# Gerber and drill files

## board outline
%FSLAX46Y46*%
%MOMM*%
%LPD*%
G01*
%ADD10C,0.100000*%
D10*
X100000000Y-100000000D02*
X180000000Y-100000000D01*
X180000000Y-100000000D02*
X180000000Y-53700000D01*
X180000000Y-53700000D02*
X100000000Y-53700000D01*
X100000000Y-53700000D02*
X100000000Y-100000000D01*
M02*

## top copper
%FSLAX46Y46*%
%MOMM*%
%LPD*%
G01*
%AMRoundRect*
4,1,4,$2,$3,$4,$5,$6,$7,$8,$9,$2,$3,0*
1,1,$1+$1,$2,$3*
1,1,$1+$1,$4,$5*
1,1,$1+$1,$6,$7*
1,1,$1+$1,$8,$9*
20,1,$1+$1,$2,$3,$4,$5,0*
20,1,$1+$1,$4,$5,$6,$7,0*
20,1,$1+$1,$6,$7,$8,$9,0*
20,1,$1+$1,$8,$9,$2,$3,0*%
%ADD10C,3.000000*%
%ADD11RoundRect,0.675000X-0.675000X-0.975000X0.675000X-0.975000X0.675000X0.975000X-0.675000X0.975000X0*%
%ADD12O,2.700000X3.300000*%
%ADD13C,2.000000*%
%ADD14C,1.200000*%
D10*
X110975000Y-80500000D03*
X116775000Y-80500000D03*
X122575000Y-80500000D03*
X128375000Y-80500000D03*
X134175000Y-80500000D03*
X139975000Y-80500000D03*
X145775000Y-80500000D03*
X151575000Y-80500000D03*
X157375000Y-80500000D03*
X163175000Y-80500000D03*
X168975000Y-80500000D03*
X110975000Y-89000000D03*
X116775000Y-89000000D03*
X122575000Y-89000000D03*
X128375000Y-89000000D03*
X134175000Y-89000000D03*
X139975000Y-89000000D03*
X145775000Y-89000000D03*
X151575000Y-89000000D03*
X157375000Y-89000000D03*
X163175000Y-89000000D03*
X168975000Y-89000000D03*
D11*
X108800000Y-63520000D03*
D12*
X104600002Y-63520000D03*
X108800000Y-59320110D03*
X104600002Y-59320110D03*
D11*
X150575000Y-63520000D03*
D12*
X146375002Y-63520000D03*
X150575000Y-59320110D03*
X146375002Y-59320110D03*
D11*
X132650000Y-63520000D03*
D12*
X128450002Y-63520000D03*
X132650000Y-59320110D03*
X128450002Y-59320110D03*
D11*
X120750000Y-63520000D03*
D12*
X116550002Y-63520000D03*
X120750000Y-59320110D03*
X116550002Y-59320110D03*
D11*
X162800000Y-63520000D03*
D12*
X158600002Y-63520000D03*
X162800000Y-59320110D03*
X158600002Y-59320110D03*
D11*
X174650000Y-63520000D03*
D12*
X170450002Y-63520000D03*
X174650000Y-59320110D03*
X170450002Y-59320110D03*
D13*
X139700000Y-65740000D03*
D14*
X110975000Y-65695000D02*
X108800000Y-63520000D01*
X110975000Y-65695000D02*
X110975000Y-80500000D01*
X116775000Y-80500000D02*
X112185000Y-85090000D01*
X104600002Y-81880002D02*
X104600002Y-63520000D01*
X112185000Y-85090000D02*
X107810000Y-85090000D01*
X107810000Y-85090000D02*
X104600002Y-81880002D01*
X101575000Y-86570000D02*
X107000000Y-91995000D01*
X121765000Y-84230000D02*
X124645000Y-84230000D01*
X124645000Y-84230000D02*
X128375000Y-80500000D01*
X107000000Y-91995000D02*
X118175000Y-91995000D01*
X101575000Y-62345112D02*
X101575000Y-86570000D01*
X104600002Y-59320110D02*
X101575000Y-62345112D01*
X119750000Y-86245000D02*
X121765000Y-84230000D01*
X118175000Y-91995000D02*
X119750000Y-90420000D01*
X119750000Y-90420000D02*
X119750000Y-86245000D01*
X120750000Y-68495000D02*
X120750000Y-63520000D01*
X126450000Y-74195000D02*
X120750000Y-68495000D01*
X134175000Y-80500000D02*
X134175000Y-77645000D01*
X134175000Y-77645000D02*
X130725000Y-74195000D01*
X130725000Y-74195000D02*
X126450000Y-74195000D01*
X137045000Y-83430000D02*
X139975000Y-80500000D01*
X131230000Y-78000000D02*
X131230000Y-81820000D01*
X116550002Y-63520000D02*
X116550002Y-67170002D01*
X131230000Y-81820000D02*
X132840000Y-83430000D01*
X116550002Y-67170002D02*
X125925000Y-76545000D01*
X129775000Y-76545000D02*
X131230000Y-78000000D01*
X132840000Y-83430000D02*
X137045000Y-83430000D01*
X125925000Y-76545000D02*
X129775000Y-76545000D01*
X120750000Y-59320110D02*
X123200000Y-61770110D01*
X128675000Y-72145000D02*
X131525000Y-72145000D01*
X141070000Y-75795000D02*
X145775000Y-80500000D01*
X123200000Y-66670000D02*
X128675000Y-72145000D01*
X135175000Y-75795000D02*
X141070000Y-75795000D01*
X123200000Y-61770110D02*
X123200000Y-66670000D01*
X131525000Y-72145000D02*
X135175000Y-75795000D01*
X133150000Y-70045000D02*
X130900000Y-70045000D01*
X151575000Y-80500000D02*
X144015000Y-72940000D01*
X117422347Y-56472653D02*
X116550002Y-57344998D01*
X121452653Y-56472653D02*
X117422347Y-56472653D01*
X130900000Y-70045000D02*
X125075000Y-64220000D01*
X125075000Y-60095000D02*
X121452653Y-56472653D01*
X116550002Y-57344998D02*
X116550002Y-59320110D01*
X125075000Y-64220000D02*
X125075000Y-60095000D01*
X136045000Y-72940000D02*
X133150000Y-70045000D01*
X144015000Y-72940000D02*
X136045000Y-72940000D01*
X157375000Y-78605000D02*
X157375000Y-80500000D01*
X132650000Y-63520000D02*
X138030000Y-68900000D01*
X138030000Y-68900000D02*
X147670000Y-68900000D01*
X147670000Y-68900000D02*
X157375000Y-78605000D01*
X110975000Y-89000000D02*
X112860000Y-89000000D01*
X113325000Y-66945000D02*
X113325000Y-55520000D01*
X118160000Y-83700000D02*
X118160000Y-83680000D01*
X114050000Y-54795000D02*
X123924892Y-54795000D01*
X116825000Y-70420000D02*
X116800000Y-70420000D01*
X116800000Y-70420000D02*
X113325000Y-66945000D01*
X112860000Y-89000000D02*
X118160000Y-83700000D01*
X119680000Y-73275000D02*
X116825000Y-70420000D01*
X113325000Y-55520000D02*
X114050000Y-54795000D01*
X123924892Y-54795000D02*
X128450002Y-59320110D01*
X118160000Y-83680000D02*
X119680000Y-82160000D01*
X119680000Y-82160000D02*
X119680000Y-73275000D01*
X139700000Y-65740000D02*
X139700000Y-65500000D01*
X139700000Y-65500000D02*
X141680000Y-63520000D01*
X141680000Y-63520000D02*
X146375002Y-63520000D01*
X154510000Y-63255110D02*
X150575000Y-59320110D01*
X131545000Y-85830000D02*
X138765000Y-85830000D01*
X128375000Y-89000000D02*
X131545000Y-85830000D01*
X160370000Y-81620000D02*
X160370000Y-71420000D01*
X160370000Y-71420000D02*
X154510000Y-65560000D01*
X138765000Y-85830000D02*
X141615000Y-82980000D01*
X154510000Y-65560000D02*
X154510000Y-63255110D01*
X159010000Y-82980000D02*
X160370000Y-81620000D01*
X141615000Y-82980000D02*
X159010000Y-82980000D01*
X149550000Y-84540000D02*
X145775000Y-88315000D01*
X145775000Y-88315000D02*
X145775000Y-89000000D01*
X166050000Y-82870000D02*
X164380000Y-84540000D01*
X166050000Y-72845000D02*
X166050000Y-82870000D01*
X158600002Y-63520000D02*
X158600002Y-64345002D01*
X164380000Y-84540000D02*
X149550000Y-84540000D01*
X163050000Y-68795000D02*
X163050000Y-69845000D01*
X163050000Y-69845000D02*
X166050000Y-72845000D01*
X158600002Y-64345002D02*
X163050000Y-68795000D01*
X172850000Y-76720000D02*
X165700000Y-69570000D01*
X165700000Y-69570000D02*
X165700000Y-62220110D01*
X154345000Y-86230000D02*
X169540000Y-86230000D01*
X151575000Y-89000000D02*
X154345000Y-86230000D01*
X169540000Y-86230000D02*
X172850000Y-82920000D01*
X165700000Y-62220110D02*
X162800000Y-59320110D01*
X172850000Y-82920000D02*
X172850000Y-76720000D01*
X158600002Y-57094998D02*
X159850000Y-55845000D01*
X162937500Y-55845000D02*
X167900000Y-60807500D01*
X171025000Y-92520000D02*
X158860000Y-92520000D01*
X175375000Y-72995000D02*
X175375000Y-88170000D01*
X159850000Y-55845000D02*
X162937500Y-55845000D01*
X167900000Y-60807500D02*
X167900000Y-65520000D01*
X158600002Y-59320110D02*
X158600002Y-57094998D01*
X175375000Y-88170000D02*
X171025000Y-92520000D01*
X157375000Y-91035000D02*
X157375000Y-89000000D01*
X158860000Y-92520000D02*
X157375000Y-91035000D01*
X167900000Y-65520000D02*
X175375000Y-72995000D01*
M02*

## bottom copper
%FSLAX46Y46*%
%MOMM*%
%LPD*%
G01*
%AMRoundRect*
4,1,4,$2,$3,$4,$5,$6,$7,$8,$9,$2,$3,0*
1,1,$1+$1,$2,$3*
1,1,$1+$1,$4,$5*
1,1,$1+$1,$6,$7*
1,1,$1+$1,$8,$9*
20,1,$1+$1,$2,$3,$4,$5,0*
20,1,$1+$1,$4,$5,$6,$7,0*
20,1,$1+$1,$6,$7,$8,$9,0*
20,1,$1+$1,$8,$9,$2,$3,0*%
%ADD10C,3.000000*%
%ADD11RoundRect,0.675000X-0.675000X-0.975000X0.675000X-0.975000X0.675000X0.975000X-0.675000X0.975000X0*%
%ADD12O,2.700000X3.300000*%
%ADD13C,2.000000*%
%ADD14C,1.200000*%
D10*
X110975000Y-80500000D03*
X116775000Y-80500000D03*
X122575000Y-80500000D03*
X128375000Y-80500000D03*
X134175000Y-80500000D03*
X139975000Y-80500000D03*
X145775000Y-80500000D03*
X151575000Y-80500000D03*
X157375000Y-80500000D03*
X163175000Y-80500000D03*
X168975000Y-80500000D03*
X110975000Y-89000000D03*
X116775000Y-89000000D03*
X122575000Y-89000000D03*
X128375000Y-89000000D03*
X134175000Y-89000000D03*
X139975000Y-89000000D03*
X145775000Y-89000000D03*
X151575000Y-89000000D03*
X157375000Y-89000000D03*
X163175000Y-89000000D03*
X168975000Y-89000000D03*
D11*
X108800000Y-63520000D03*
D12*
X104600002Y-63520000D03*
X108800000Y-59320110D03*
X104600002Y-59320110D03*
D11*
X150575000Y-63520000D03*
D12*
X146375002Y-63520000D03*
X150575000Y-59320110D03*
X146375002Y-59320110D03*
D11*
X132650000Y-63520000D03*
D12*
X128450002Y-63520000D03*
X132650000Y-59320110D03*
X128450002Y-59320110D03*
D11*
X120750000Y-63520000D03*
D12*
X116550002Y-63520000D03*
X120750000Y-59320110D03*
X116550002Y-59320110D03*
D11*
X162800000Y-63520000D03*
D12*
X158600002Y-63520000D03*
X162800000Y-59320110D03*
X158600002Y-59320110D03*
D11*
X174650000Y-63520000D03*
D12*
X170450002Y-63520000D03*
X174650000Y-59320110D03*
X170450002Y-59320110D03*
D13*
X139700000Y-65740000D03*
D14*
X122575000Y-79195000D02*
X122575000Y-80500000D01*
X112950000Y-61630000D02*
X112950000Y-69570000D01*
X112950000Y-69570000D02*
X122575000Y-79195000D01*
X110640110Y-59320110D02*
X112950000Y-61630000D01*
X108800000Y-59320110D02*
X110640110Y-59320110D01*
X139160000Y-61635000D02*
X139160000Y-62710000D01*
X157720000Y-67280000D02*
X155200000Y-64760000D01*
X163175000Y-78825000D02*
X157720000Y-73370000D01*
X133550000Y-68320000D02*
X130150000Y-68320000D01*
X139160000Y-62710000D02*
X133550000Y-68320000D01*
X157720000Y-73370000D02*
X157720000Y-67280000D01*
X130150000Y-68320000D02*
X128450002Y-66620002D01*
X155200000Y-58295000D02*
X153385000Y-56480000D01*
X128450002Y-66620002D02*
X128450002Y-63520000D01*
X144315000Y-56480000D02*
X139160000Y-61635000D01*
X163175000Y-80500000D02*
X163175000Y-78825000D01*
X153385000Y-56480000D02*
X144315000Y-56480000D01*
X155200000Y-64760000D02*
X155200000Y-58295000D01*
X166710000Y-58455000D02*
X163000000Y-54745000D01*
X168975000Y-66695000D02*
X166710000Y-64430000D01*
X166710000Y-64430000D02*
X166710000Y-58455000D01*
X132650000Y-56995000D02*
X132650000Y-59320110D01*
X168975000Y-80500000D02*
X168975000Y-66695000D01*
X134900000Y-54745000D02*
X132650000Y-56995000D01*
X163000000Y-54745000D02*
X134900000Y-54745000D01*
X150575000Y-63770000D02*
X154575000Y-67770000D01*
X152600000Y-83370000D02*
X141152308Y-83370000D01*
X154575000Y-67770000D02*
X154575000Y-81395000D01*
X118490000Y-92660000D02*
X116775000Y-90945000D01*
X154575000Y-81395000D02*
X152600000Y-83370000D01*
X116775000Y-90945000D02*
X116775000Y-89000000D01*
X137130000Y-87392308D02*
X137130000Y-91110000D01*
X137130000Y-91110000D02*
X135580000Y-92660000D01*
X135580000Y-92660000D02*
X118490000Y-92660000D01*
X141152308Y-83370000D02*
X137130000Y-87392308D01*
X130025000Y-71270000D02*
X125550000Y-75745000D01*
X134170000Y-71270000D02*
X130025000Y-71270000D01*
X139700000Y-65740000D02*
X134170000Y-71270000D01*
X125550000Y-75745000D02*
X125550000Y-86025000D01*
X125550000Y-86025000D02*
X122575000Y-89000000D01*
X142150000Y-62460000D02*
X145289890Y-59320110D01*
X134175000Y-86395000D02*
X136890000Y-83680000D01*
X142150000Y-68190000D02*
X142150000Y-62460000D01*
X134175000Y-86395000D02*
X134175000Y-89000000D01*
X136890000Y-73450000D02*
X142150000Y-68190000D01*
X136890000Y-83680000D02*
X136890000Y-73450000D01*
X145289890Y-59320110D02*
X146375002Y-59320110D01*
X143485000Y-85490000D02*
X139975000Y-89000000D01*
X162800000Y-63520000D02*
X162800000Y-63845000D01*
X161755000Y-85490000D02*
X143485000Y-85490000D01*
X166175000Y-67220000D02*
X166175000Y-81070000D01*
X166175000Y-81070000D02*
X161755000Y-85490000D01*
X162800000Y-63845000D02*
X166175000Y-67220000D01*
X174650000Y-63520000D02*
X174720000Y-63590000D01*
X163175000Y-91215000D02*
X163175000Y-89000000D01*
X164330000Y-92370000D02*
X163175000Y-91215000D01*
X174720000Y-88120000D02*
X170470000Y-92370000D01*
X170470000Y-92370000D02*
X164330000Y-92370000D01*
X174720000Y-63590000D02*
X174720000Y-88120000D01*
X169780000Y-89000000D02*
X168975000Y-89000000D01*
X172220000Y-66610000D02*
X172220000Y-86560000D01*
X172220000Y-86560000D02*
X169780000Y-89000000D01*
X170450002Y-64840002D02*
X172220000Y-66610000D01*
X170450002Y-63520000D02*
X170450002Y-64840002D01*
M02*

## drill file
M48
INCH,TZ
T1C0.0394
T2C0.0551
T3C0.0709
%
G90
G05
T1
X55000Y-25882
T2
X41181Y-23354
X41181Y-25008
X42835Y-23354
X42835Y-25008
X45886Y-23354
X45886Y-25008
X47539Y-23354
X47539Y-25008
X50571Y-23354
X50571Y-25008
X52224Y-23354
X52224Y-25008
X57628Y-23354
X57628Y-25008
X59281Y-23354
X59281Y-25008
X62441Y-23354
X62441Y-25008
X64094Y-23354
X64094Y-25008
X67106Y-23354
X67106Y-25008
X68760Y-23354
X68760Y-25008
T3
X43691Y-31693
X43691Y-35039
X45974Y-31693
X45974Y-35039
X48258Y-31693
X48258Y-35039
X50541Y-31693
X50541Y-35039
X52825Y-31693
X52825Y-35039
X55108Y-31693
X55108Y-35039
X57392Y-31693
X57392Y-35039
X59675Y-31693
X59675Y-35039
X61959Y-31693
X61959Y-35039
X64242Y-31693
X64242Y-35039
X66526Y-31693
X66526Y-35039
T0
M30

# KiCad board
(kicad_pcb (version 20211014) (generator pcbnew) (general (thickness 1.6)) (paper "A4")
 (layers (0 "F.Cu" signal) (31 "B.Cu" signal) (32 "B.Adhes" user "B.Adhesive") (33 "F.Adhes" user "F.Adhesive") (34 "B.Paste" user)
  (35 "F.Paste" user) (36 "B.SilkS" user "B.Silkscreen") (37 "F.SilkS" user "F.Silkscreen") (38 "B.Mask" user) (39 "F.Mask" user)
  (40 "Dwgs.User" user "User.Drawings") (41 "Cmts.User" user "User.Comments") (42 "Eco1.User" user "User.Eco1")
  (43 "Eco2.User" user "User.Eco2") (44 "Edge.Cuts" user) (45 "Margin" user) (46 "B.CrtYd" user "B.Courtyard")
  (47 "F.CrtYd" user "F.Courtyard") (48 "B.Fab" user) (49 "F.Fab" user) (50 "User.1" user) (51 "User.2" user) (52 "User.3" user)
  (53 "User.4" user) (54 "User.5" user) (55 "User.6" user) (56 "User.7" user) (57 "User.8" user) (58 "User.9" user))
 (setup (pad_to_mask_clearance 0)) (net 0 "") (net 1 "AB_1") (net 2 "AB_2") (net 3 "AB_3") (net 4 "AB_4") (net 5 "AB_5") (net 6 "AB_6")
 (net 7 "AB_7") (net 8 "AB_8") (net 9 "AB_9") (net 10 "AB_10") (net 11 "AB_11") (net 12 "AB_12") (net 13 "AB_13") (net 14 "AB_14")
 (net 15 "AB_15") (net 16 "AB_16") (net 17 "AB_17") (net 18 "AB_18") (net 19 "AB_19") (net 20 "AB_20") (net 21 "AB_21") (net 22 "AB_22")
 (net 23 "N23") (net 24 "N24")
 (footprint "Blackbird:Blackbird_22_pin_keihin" (layer "F.Cu") (at 110.975 80.5)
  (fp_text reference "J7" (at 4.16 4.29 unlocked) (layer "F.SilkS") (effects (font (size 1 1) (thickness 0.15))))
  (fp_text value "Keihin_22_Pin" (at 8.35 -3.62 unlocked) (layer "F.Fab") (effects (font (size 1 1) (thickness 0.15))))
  (pad "1" thru_hole circle (at 0 0) (size 3 3) (drill 1.8) (layers *.Cu *.Mask) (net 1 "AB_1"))
  (pad "2" thru_hole circle (at 5.8 0) (size 3 3) (drill 1.8) (layers *.Cu *.Mask) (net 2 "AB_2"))
  (pad "3" thru_hole circle (at 11.6 0) (size 3 3) (drill 1.8) (layers *.Cu *.Mask) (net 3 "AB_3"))
  (pad "4" thru_hole circle (at 17.4 0) (size 3 3) (drill 1.8) (layers *.Cu *.Mask) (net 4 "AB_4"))
  (pad "5" thru_hole circle (at 23.2 0) (size 3 3) (drill 1.8) (layers *.Cu *.Mask) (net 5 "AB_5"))
  (pad "6" thru_hole circle (at 29 0) (size 3 3) (drill 1.8) (layers *.Cu *.Mask) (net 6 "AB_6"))
  (pad "7" thru_hole circle (at 34.8 0) (size 3 3) (drill 1.8) (layers *.Cu *.Mask) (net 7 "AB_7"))
  (pad "8" thru_hole circle (at 40.6 0) (size 3 3) (drill 1.8) (layers *.Cu *.Mask) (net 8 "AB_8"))
  (pad "9" thru_hole circle (at 46.4 0) (size 3 3) (drill 1.8) (layers *.Cu *.Mask) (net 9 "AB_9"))
  (pad "10" thru_hole circle (at 52.2 0) (size 3 3) (drill 1.8) (layers *.Cu *.Mask) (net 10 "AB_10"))
  (pad "11" thru_hole circle (at 58 0) (size 3 3) (drill 1.8) (layers *.Cu *.Mask) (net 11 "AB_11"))
  (pad "12" thru_hole circle (at 0 8.5) (size 3 3) (drill 1.8) (layers *.Cu *.Mask) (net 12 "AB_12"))
  (pad "13" thru_hole circle (at 5.8 8.5) (size 3 3) (drill 1.8) (layers *.Cu *.Mask) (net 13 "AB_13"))
  (pad "14" thru_hole circle (at 11.6 8.5) (size 3 3) (drill 1.8) (layers *.Cu *.Mask) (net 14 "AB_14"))
  (pad "15" thru_hole circle (at 17.4 8.5) (size 3 3) (drill 1.8) (layers *.Cu *.Mask) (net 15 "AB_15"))
  (pad "16" thru_hole circle (at 23.2 8.5) (size 3 3) (drill 1.8) (layers *.Cu *.Mask) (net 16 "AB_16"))
  (pad "17" thru_hole circle (at 29 8.5) (size 3 3) (drill 1.8) (layers *.Cu *.Mask) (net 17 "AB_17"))
  (pad "18" thru_hole circle (at 34.8 8.5) (size 3 3) (drill 1.8) (layers *.Cu *.Mask) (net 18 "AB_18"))
  (pad "19" thru_hole circle (at 40.6 8.5) (size 3 3) (drill 1.8) (layers *.Cu *.Mask) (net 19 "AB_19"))
  (pad "20" thru_hole circle (at 46.4 8.5) (size 3 3) (drill 1.8) (layers *.Cu *.Mask) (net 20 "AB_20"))
  (pad "21" thru_hole circle (at 52.2 8.5) (size 3 3) (drill 1.8) (layers *.Cu *.Mask) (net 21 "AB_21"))
  (pad "22" thru_hole circle (at 58 8.5) (size 3 3) (drill 1.8) (layers *.Cu *.Mask) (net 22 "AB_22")))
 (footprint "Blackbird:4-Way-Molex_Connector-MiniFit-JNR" (layer "F.Cu") (at 108.8 63.52)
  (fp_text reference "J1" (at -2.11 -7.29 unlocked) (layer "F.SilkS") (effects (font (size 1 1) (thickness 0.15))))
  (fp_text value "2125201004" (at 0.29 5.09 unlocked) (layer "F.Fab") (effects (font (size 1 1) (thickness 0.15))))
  (pad "1" thru_hole roundrect (at 0 0) (size 2.7 3.3) (drill 1.4) (layers *.Cu *.Mask) (roundrect_rratio 0.25) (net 1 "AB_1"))
  (pad "2" thru_hole oval (at -4.199998 0) (size 2.7 3.3) (drill 1.4) (layers *.Cu *.Mask) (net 2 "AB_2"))
  (pad "3" thru_hole oval (at 0 -4.19989) (size 2.7 3.3) (drill 1.4) (layers *.Cu *.Mask) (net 3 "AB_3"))
  (pad "4" thru_hole oval (at -4.199998 -4.19989) (size 2.7 3.3) (drill 1.4) (layers *.Cu *.Mask) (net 4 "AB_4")))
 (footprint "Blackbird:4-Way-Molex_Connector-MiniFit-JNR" (layer "F.Cu") (at 150.575 63.52)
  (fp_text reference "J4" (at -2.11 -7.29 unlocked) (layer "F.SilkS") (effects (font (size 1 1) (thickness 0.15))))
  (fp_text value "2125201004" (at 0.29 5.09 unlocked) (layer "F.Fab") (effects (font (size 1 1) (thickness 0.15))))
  (pad "1" thru_hole roundrect (at 0 0) (size 2.7 3.3) (drill 1.4) (layers *.Cu *.Mask) (roundrect_rratio 0.25) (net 13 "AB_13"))
  (pad "2" thru_hole oval (at -4.199998 0) (size 2.7 3.3) (drill 1.4) (layers *.Cu *.Mask) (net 14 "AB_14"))
  (pad "3" thru_hole oval (at 0 -4.19989) (size 2.7 3.3) (drill 1.4) (layers *.Cu *.Mask) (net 15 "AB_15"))
  (pad "4" thru_hole oval (at -4.199998 -4.19989) (size 2.7 3.3) (drill 1.4) (layers *.Cu *.Mask) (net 16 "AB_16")))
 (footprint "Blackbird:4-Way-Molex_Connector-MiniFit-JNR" (layer "F.Cu") (at 132.65 63.52)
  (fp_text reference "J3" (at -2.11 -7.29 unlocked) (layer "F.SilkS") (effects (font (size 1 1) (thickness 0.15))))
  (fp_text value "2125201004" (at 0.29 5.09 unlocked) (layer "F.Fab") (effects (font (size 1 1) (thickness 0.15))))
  (pad "1" thru_hole roundrect (at 0 0) (size 2.7 3.3) (drill 1.4) (layers *.Cu *.Mask) (roundrect_rratio 0.25) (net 9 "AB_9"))
  (pad "2" thru_hole oval (at -4.199998 0) (size 2.7 3.3) (drill 1.4) (layers *.Cu *.Mask) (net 10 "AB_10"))
  (pad "3" thru_hole oval (at 0 -4.19989) (size 2.7 3.3) (drill 1.4) (layers *.Cu *.Mask) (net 11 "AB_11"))
  (pad "4" thru_hole oval (at -4.199998 -4.19989) (size 2.7 3.3) (drill 1.4) (layers *.Cu *.Mask) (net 12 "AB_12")))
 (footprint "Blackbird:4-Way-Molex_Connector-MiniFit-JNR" (layer "F.Cu") (at 120.75 63.52)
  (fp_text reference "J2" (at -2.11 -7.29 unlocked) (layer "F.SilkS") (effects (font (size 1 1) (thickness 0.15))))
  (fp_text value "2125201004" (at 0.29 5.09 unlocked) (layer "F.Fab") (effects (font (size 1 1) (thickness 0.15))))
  (pad "1" thru_hole roundrect (at 0 0) (size 2.7 3.3) (drill 1.4) (layers *.Cu *.Mask) (roundrect_rratio 0.25) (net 5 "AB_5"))
  (pad "2" thru_hole oval (at -4.199998 0) (size 2.7 3.3) (drill 1.4) (layers *.Cu *.Mask) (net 6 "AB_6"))
  (pad "3" thru_hole oval (at 0 -4.19989) (size 2.7 3.3) (drill 1.4) (layers *.Cu *.Mask) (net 7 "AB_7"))
  (pad "4" thru_hole oval (at -4.199998 -4.19989) (size 2.7 3.3) (drill 1.4) (layers *.Cu *.Mask) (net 8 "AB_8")))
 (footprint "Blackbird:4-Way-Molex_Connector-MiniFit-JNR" (layer "F.Cu") (at 162.8 63.52)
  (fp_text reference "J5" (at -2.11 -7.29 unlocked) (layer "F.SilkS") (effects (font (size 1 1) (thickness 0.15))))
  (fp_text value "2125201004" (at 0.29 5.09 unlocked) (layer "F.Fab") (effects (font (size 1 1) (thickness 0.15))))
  (pad "1" thru_hole roundrect (at 0 0) (size 2.7 3.3) (drill 1.4) (layers *.Cu *.Mask) (roundrect_rratio 0.25) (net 17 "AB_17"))
  (pad "2" thru_hole oval (at -4.199998 0) (size 2.7 3.3) (drill 1.4) (layers *.Cu *.Mask) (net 18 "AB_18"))
  (pad "3" thru_hole oval (at 0 -4.19989) (size 2.7 3.3) (drill 1.4) (layers *.Cu *.Mask) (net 19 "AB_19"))
  (pad "4" thru_hole oval (at -4.199998 -4.19989) (size 2.7 3.3) (drill 1.4) (layers *.Cu *.Mask) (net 20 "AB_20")))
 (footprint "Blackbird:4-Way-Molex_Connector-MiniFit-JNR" (layer "F.Cu") (at 174.65 63.52)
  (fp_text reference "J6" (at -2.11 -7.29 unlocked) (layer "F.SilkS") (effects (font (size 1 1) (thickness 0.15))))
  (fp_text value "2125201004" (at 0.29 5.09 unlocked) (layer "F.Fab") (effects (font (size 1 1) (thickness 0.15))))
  (pad "1" thru_hole roundrect (at 0 0) (size 2.7 3.3) (drill 1.4) (layers *.Cu *.Mask) (roundrect_rratio 0.25) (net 21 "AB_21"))
  (pad "2" thru_hole oval (at -4.199998 0) (size 2.7 3.3) (drill 1.4) (layers *.Cu *.Mask) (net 22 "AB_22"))
  (pad "3" thru_hole oval (at 0 -4.19989) (size 2.7 3.3) (drill 1.4) (layers *.Cu *.Mask) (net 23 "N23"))
  (pad "4" thru_hole oval (at -4.199998 -4.19989) (size 2.7 3.3) (drill 1.4) (layers *.Cu *.Mask) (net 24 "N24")))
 (gr_rect (start 100 100) (end 180 53.7) (layer "Edge.Cuts") (width 0.1) (fill none))
 (segment (start 110.975 65.695) (end 108.8 63.52) (width 1.2) (layer "F.Cu") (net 1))
 (segment (start 110.975 65.695) (end 110.975 80.5) (width 1.2) (layer "F.Cu") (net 1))
 (segment (start 116.775 80.5) (end 112.185 85.09) (width 1.2) (layer "F.Cu") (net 2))
 (segment (start 104.600002 81.880002) (end 104.600002 63.52) (width 1.2) (layer "F.Cu") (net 2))
 (segment (start 112.185 85.09) (end 107.81 85.09) (width 1.2) (layer "F.Cu") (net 2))
 (segment (start 107.81 85.09) (end 104.600002 81.880002) (width 1.2) (layer "F.Cu") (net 2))
 (segment (start 122.575 79.195) (end 122.575 80.5) (width 1.2) (layer "B.Cu") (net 3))
 (segment (start 112.95 61.63) (end 112.95 69.57) (width 1.2) (layer "B.Cu") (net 3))
 (segment (start 112.95 69.57) (end 122.575 79.195) (width 1.2) (layer "B.Cu") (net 3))
 (segment (start 110.64011 59.32011) (end 112.95 61.63) (width 1.2) (layer "B.Cu") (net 3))
 (segment (start 108.8 59.32011) (end 110.64011 59.32011) (width 1.2) (layer "B.Cu") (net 3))
 (segment (start 101.575 86.57) (end 107 91.995) (width 1.2) (layer "F.Cu") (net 4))
 (segment (start 121.765 84.23) (end 124.645 84.23) (width 1.2) (layer "F.Cu") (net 4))
 (segment (start 124.645 84.23) (end 128.375 80.5) (width 1.2) (layer "F.Cu") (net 4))
 (segment (start 107 91.995) (end 118.175 91.995) (width 1.2) (layer "F.Cu") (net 4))
 (segment (start 101.575 62.345112) (end 101.575 86.57) (width 1.2) (layer "F.Cu") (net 4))
 (segment (start 104.600002 59.32011) (end 101.575 62.345112) (width 1.2) (layer "F.Cu") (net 4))
 (segment (start 119.75 86.245) (end 121.765 84.23) (width 1.2) (layer "F.Cu") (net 4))
 (segment (start 118.175 91.995) (end 119.75 90.42) (width 1.2) (layer "F.Cu") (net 4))
 (segment (start 119.75 90.42) (end 119.75 86.245) (width 1.2) (layer "F.Cu") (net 4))
 (segment (start 120.75 68.495) (end 120.75 63.52) (width 1.2) (layer "F.Cu") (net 5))
 (segment (start 126.45 74.195) (end 120.75 68.495) (width 1.2) (layer "F.Cu") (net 5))
 (segment (start 134.175 80.5) (end 134.175 77.645) (width 1.2) (layer "F.Cu") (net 5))
 (segment (start 134.175 77.645) (end 130.725 74.195) (width 1.2) (layer "F.Cu") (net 5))
 (segment (start 130.725 74.195) (end 126.45 74.195) (width 1.2) (layer "F.Cu") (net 5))
 (segment (start 137.045 83.43) (end 139.975 80.5) (width 1.2) (layer "F.Cu") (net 6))
 (segment (start 131.23 78) (end 131.23 81.82) (width 1.2) (layer "F.Cu") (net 6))
 (segment (start 116.550002 63.52) (end 116.550002 67.170002) (width 1.2) (layer "F.Cu") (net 6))
 (segment (start 131.23 81.82) (end 132.84 83.43) (width 1.2) (layer "F.Cu") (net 6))
 (segment (start 116.550002 67.170002) (end 125.925 76.545) (width 1.2) (layer "F.Cu") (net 6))
 (segment (start 129.775 76.545) (end 131.23 78) (width 1.2) (layer "F.Cu") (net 6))
 (segment (start 132.84 83.43) (end 137.045 83.43) (width 1.2) (layer "F.Cu") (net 6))
 (segment (start 125.925 76.545) (end 129.775 76.545) (width 1.2) (layer "F.Cu") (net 6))
 (segment (start 120.75 59.32011) (end 123.2 61.77011) (width 1.2) (layer "F.Cu") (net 7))
 (segment (start 128.675 72.145) (end 131.525 72.145) (width 1.2) (layer "F.Cu") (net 7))
 (segment (start 141.07 75.795) (end 145.775 80.5) (width 1.2) (layer "F.Cu") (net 7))
 (segment (start 123.2 66.67) (end 128.675 72.145) (width 1.2) (layer "F.Cu") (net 7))
 (segment (start 135.175 75.795) (end 141.07 75.795) (width 1.2) (layer "F.Cu") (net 7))
 (segment (start 123.2 61.77011) (end 123.2 66.67) (width 1.2) (layer "F.Cu") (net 7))
 (segment (start 131.525 72.145) (end 135.175 75.795) (width 1.2) (layer "F.Cu") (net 7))
 (segment (start 133.15 70.045) (end 130.9 70.045) (width 1.2) (layer "F.Cu") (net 8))
 (segment (start 151.575 80.5) (end 144.015 72.94) (width 1.2) (layer "F.Cu") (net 8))
 (segment (start 117.422347 56.472653) (end 116.550002 57.344998) (width 1.2) (layer "F.Cu") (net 8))
 (segment (start 121.452653 56.472653) (end 117.422347 56.472653) (width 1.2) (layer "F.Cu") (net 8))
 (segment (start 130.9 70.045) (end 125.075 64.22) (width 1.2) (layer "F.Cu") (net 8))
 (segment (start 125.075 60.095) (end 121.452653 56.472653) (width 1.2) (layer "F.Cu") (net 8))
 (segment (start 116.550002 57.344998) (end 116.550002 59.32011) (width 1.2) (layer "F.Cu") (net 8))
 (segment (start 125.075 64.22) (end 125.075 60.095) (width 1.2) (layer "F.Cu") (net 8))
 (segment (start 136.045 72.94) (end 133.15 70.045) (width 1.2) (layer "F.Cu") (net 8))
 (segment (start 144.015 72.94) (end 136.045 72.94) (width 1.2) (layer "F.Cu") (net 8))
 (segment (start 157.375 78.605) (end 157.375 80.5) (width 1.2) (layer "F.Cu") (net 9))
 (segment (start 132.65 63.52) (end 138.03 68.9) (width 1.2) (layer "F.Cu") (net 9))
 (segment (start 138.03 68.9) (end 147.67 68.9) (width 1.2) (layer "F.Cu") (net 9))
 (segment (start 147.67 68.9) (end 157.375 78.605) (width 1.2) (layer "F.Cu") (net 9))
 (segment (start 139.16 61.635) (end 139.16 62.71) (width 1.2) (layer "B.Cu") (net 10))
 (segment (start 157.72 67.28) (end 155.2 64.76) (width 1.2) (layer "B.Cu") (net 10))
 (segment (start 163.175 78.825) (end 157.72 73.37) (width 1.2) (layer "B.Cu") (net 10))
 (segment (start 133.55 68.32) (end 130.15 68.32) (width 1.2) (layer "B.Cu") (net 10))
 (segment (start 139.16 62.71) (end 133.55 68.32) (width 1.2) (layer "B.Cu") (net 10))
 (segment (start 157.72 73.37) (end 157.72 67.28) (width 1.2) (layer "B.Cu") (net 10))
 (segment (start 130.15 68.32) (end 128.450002 66.620002) (width 1.2) (layer "B.Cu") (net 10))
 (segment (start 155.2 58.295) (end 153.385 56.48) (width 1.2) (layer "B.Cu") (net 10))
 (segment (start 128.450002 66.620002) (end 128.450002 63.52) (width 1.2) (layer "B.Cu") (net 10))
 (segment (start 144.315 56.48) (end 139.16 61.635) (width 1.2) (layer "B.Cu") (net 10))
 (segment (start 163.175 80.5) (end 163.175 78.825) (width 1.2) (layer "B.Cu") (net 10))
 (segment (start 153.385 56.48) (end 144.315 56.48) (width 1.2) (layer "B.Cu") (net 10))
 (segment (start 155.2 64.76) (end 155.2 58.295) (width 1.2) (layer "B.Cu") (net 10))
 (segment (start 166.71 58.455) (end 163 54.745) (width 1.2) (layer "B.Cu") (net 11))
 (segment (start 168.975 66.695) (end 166.71 64.43) (width 1.2) (layer "B.Cu") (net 11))
 (segment (start 166.71 64.43) (end 166.71 58.455) (width 1.2) (layer "B.Cu") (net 11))
 (segment (start 132.65 56.995) (end 132.65 59.32011) (width 1.2) (layer "B.Cu") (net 11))
 (segment (start 168.975 80.5) (end 168.975 66.695) (width 1.2) (layer "B.Cu") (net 11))
 (segment (start 134.9 54.745) (end 132.65 56.995) (width 1.2) (layer "B.Cu") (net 11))
 (segment (start 163 54.745) (end 134.9 54.745) (width 1.2) (layer "B.Cu") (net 11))
 (segment (start 110.975 89) (end 112.86 89) (width 1.2) (layer "F.Cu") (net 12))
 (segment (start 113.325 66.945) (end 113.325 55.52) (width 1.2) (layer "F.Cu") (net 12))
 (segment (start 118.16 83.7) (end 118.16 83.68) (width 1.2) (layer "F.Cu") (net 12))
 (segment (start 114.05 54.795) (end 123.924892 54.795) (width 1.2) (layer "F.Cu") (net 12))
 (segment (start 116.825 70.42) (end 116.8 70.42) (width 1.2) (layer "F.Cu") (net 12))
 (segment (start 116.8 70.42) (end 113.325 66.945) (width 1.2) (layer "F.Cu") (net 12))
 (segment (start 112.86 89) (end 118.16 83.7) (width 1.2) (layer "F.Cu") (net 12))
 (segment (start 119.68 73.275) (end 116.825 70.42) (width 1.2) (layer "F.Cu") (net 12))
 (segment (start 113.325 55.52) (end 114.05 54.795) (width 1.2) (layer "F.Cu") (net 12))
 (segment (start 123.924892 54.795) (end 128.450002 59.32011) (width 1.2) (layer "F.Cu") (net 12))
 (segment (start 118.16 83.68) (end 119.68 82.16) (width 1.2) (layer "F.Cu") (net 12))
 (segment (start 119.68 82.16) (end 119.68 73.275) (width 1.2) (layer "F.Cu") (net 12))
 (segment (start 150.575 63.77) (end 154.575 67.77) (width 1.2) (layer "B.Cu") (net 13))
 (segment (start 152.6 83.37) (end 141.152308 83.37) (width 1.2) (layer "B.Cu") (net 13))
 (segment (start 154.575 67.77) (end 154.575 81.395) (width 1.2) (layer "B.Cu") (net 13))
 (segment (start 118.49 92.66) (end 116.775 90.945) (width 1.2) (layer "B.Cu") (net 13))
 (segment (start 154.575 81.395) (end 152.6 83.37) (width 1.2) (layer "B.Cu") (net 13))
 (segment (start 116.775 90.945) (end 116.775 89) (width 1.2) (layer "B.Cu") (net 13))
 (segment (start 137.13 87.392308) (end 137.13 91.11) (width 1.2) (layer "B.Cu") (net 13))
 (segment (start 137.13 91.11) (end 135.58 92.66) (width 1.2) (layer "B.Cu") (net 13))
 (segment (start 135.58 92.66) (end 118.49 92.66) (width 1.2) (layer "B.Cu") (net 13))
 (segment (start 141.152308 83.37) (end 137.13 87.392308) (width 1.2) (layer "B.Cu") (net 13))
 (segment (start 139.7 65.74) (end 139.7 65.5) (width 1.2) (layer "F.Cu") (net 14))
 (segment (start 139.7 65.5) (end 141.68 63.52) (width 1.2) (layer "F.Cu") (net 14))
 (segment (start 141.68 63.52) (end 146.375002 63.52) (width 1.2) (layer "F.Cu") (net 14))
 (via (at 139.7 65.74) (size 2) (drill 1) (layers "F.Cu" "B.Cu") (free) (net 14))
 (segment (start 130.025 71.27) (end 125.55 75.745) (width 1.2) (layer "B.Cu") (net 14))
 (segment (start 134.17 71.27) (end 130.025 71.27) (width 1.2) (layer "B.Cu") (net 14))
 (segment (start 139.7 65.74) (end 134.17 71.27) (width 1.2) (layer "B.Cu") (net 14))
 (segment (start 125.55 75.745) (end 125.55 86.025) (width 1.2) (layer "B.Cu") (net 14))
 (segment (start 125.55 86.025) (end 122.575 89) (width 1.2) (layer "B.Cu") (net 14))
 (segment (start 154.51 63.25511) (end 150.575 59.32011) (width 1.2) (layer "F.Cu") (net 15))
 (segment (start 131.545 85.83) (end 138.765 85.83) (width 1.2) (layer "F.Cu") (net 15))
 (segment (start 128.375 89) (end 131.545 85.83) (width 1.2) (layer "F.Cu") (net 15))
 (segment (start 160.37 81.62) (end 160.37 71.42) (width 1.2) (layer "F.Cu") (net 15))
 (segment (start 160.37 71.42) (end 154.51 65.56) (width 1.2) (layer "F.Cu") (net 15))
 (segment (start 138.765 85.83) (end 141.615 82.98) (width 1.2) (layer "F.Cu") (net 15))
 (segment (start 154.51 65.56) (end 154.51 63.25511) (width 1.2) (layer "F.Cu") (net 15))
 (segment (start 159.01 82.98) (end 160.37 81.62) (width 1.2) (layer "F.Cu") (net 15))
 (segment (start 141.615 82.98) (end 159.01 82.98) (width 1.2) (layer "F.Cu") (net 15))
 (segment (start 142.15 62.46) (end 145.28989 59.32011) (width 1.2) (layer "B.Cu") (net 16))
 (segment (start 134.175 86.395) (end 136.89 83.68) (width 1.2) (layer "B.Cu") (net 16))
 (segment (start 142.15 68.19) (end 142.15 62.46) (width 1.2) (layer "B.Cu") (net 16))
 (segment (start 134.175 86.395) (end 134.175 89) (width 1.2) (layer "B.Cu") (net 16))
 (segment (start 136.89 73.45) (end 142.15 68.19) (width 1.2) (layer "B.Cu") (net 16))
 (segment (start 136.89 83.68) (end 136.89 73.45) (width 1.2) (layer "B.Cu") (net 16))
 (segment (start 145.28989 59.32011) (end 146.375002 59.32011) (width 1.2) (layer "B.Cu") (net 16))
 (segment (start 143.485 85.49) (end 139.975 89) (width 1.2) (layer "B.Cu") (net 17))
 (segment (start 162.8 63.52) (end 162.8 63.845) (width 1.2) (layer "B.Cu") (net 17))
 (segment (start 161.755 85.49) (end 143.485 85.49) (width 1.2) (layer "B.Cu") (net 17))
 (segment (start 166.175 67.22) (end 166.175 81.07) (width 1.2) (layer "B.Cu") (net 17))
 (segment (start 166.175 81.07) (end 161.755 85.49) (width 1.2) (layer "B.Cu") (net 17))
 (segment (start 162.8 63.845) (end 166.175 67.22) (width 1.2) (layer "B.Cu") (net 17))
 (segment (start 149.55 84.54) (end 145.775 88.315) (width 1.2) (layer "F.Cu") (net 18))
 (segment (start 145.775 88.315) (end 145.775 89) (width 1.2) (layer "F.Cu") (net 18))
 (segment (start 166.05 82.87) (end 164.38 84.54) (width 1.2) (layer "F.Cu") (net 18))
 (segment (start 166.05 72.845) (end 166.05 82.87) (width 1.2) (layer "F.Cu") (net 18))
 (segment (start 158.600002 63.52) (end 158.600002 64.345002) (width 1.2) (layer "F.Cu") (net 18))
 (segment (start 164.38 84.54) (end 149.55 84.54) (width 1.2) (layer "F.Cu") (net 18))
 (segment (start 163.05 68.795) (end 163.05 69.845) (width 1.2) (layer "F.Cu") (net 18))
 (segment (start 163.05 69.845) (end 166.05 72.845) (width 1.2) (layer "F.Cu") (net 18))
 (segment (start 158.600002 64.345002) (end 163.05 68.795) (width 1.2) (layer "F.Cu") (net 18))
 (segment (start 172.85 76.72) (end 165.7 69.57) (width 1.2) (layer "F.Cu") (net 19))
 (segment (start 165.7 69.57) (end 165.7 62.22011) (width 1.2) (layer "F.Cu") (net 19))
 (segment (start 154.345 86.23) (end 169.54 86.23) (width 1.2) (layer "F.Cu") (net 19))
 (segment (start 151.575 89) (end 154.345 86.23) (width 1.2) (layer "F.Cu") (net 19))
 (segment (start 169.54 86.23) (end 172.85 82.92) (width 1.2) (layer "F.Cu") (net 19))
 (segment (start 165.7 62.22011) (end 162.8 59.32011) (width 1.2) (layer "F.Cu") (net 19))
 (segment (start 172.85 82.92) (end 172.85 76.72) (width 1.2) (layer "F.Cu") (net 19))
 (segment (start 158.600002 57.094998) (end 159.85 55.845) (width 1.2) (layer "F.Cu") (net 20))
 (segment (start 162.9375 55.845) (end 167.9 60.8075) (width 1.2) (layer "F.Cu") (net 20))
 (segment (start 171.025 92.52) (end 158.86 92.52) (width 1.2) (layer "F.Cu") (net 20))
 (segment (start 175.375 72.995) (end 175.375 88.17) (width 1.2) (layer "F.Cu") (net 20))
 (segment (start 159.85 55.845) (end 162.9375 55.845) (width 1.2) (layer "F.Cu") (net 20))
 (segment (start 167.9 60.8075) (end 167.9 65.52) (width 1.2) (layer "F.Cu") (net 20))
 (segment (start 158.600002 59.32011) (end 158.600002 57.094998) (width 1.2) (layer "F.Cu") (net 20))
 (segment (start 175.375 88.17) (end 171.025 92.52) (width 1.2) (layer "F.Cu") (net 20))
 (segment (start 157.375 91.035) (end 157.375 89) (width 1.2) (layer "F.Cu") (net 20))
 (segment (start 158.86 92.52) (end 157.375 91.035) (width 1.2) (layer "F.Cu") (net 20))
 (segment (start 167.9 65.52) (end 175.375 72.995) (width 1.2) (layer "F.Cu") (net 20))
 (segment (start 174.65 63.52) (end 174.72 63.59) (width 1.2) (layer "B.Cu") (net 21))
 (segment (start 163.175 91.215) (end 163.175 89) (width 1.2) (layer "B.Cu") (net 21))
 (segment (start 164.33 92.37) (end 163.175 91.215) (width 1.2) (layer "B.Cu") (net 21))
 (segment (start 174.72 88.12) (end 170.47 92.37) (width 1.2) (layer "B.Cu") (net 21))
 (segment (start 170.47 92.37) (end 164.33 92.37) (width 1.2) (layer "B.Cu") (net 21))
 (segment (start 174.72 63.59) (end 174.72 88.12) (width 1.2) (layer "B.Cu") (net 21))
 (segment (start 169.78 89) (end 168.975 89) (width 1.2) (layer "B.Cu") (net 22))
 (segment (start 172.22 66.61) (end 172.22 86.56) (width 1.2) (layer "B.Cu") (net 22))
 (segment (start 172.22 86.56) (end 169.78 89) (width 1.2) (layer "B.Cu") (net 22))
 (segment (start 170.450002 64.840002) (end 172.22 66.61) (width 1.2) (layer "B.Cu") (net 22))
 (segment (start 170.450002 63.52) (end 170.450002 64.840002) (width 1.2) (layer "B.Cu") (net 22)))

